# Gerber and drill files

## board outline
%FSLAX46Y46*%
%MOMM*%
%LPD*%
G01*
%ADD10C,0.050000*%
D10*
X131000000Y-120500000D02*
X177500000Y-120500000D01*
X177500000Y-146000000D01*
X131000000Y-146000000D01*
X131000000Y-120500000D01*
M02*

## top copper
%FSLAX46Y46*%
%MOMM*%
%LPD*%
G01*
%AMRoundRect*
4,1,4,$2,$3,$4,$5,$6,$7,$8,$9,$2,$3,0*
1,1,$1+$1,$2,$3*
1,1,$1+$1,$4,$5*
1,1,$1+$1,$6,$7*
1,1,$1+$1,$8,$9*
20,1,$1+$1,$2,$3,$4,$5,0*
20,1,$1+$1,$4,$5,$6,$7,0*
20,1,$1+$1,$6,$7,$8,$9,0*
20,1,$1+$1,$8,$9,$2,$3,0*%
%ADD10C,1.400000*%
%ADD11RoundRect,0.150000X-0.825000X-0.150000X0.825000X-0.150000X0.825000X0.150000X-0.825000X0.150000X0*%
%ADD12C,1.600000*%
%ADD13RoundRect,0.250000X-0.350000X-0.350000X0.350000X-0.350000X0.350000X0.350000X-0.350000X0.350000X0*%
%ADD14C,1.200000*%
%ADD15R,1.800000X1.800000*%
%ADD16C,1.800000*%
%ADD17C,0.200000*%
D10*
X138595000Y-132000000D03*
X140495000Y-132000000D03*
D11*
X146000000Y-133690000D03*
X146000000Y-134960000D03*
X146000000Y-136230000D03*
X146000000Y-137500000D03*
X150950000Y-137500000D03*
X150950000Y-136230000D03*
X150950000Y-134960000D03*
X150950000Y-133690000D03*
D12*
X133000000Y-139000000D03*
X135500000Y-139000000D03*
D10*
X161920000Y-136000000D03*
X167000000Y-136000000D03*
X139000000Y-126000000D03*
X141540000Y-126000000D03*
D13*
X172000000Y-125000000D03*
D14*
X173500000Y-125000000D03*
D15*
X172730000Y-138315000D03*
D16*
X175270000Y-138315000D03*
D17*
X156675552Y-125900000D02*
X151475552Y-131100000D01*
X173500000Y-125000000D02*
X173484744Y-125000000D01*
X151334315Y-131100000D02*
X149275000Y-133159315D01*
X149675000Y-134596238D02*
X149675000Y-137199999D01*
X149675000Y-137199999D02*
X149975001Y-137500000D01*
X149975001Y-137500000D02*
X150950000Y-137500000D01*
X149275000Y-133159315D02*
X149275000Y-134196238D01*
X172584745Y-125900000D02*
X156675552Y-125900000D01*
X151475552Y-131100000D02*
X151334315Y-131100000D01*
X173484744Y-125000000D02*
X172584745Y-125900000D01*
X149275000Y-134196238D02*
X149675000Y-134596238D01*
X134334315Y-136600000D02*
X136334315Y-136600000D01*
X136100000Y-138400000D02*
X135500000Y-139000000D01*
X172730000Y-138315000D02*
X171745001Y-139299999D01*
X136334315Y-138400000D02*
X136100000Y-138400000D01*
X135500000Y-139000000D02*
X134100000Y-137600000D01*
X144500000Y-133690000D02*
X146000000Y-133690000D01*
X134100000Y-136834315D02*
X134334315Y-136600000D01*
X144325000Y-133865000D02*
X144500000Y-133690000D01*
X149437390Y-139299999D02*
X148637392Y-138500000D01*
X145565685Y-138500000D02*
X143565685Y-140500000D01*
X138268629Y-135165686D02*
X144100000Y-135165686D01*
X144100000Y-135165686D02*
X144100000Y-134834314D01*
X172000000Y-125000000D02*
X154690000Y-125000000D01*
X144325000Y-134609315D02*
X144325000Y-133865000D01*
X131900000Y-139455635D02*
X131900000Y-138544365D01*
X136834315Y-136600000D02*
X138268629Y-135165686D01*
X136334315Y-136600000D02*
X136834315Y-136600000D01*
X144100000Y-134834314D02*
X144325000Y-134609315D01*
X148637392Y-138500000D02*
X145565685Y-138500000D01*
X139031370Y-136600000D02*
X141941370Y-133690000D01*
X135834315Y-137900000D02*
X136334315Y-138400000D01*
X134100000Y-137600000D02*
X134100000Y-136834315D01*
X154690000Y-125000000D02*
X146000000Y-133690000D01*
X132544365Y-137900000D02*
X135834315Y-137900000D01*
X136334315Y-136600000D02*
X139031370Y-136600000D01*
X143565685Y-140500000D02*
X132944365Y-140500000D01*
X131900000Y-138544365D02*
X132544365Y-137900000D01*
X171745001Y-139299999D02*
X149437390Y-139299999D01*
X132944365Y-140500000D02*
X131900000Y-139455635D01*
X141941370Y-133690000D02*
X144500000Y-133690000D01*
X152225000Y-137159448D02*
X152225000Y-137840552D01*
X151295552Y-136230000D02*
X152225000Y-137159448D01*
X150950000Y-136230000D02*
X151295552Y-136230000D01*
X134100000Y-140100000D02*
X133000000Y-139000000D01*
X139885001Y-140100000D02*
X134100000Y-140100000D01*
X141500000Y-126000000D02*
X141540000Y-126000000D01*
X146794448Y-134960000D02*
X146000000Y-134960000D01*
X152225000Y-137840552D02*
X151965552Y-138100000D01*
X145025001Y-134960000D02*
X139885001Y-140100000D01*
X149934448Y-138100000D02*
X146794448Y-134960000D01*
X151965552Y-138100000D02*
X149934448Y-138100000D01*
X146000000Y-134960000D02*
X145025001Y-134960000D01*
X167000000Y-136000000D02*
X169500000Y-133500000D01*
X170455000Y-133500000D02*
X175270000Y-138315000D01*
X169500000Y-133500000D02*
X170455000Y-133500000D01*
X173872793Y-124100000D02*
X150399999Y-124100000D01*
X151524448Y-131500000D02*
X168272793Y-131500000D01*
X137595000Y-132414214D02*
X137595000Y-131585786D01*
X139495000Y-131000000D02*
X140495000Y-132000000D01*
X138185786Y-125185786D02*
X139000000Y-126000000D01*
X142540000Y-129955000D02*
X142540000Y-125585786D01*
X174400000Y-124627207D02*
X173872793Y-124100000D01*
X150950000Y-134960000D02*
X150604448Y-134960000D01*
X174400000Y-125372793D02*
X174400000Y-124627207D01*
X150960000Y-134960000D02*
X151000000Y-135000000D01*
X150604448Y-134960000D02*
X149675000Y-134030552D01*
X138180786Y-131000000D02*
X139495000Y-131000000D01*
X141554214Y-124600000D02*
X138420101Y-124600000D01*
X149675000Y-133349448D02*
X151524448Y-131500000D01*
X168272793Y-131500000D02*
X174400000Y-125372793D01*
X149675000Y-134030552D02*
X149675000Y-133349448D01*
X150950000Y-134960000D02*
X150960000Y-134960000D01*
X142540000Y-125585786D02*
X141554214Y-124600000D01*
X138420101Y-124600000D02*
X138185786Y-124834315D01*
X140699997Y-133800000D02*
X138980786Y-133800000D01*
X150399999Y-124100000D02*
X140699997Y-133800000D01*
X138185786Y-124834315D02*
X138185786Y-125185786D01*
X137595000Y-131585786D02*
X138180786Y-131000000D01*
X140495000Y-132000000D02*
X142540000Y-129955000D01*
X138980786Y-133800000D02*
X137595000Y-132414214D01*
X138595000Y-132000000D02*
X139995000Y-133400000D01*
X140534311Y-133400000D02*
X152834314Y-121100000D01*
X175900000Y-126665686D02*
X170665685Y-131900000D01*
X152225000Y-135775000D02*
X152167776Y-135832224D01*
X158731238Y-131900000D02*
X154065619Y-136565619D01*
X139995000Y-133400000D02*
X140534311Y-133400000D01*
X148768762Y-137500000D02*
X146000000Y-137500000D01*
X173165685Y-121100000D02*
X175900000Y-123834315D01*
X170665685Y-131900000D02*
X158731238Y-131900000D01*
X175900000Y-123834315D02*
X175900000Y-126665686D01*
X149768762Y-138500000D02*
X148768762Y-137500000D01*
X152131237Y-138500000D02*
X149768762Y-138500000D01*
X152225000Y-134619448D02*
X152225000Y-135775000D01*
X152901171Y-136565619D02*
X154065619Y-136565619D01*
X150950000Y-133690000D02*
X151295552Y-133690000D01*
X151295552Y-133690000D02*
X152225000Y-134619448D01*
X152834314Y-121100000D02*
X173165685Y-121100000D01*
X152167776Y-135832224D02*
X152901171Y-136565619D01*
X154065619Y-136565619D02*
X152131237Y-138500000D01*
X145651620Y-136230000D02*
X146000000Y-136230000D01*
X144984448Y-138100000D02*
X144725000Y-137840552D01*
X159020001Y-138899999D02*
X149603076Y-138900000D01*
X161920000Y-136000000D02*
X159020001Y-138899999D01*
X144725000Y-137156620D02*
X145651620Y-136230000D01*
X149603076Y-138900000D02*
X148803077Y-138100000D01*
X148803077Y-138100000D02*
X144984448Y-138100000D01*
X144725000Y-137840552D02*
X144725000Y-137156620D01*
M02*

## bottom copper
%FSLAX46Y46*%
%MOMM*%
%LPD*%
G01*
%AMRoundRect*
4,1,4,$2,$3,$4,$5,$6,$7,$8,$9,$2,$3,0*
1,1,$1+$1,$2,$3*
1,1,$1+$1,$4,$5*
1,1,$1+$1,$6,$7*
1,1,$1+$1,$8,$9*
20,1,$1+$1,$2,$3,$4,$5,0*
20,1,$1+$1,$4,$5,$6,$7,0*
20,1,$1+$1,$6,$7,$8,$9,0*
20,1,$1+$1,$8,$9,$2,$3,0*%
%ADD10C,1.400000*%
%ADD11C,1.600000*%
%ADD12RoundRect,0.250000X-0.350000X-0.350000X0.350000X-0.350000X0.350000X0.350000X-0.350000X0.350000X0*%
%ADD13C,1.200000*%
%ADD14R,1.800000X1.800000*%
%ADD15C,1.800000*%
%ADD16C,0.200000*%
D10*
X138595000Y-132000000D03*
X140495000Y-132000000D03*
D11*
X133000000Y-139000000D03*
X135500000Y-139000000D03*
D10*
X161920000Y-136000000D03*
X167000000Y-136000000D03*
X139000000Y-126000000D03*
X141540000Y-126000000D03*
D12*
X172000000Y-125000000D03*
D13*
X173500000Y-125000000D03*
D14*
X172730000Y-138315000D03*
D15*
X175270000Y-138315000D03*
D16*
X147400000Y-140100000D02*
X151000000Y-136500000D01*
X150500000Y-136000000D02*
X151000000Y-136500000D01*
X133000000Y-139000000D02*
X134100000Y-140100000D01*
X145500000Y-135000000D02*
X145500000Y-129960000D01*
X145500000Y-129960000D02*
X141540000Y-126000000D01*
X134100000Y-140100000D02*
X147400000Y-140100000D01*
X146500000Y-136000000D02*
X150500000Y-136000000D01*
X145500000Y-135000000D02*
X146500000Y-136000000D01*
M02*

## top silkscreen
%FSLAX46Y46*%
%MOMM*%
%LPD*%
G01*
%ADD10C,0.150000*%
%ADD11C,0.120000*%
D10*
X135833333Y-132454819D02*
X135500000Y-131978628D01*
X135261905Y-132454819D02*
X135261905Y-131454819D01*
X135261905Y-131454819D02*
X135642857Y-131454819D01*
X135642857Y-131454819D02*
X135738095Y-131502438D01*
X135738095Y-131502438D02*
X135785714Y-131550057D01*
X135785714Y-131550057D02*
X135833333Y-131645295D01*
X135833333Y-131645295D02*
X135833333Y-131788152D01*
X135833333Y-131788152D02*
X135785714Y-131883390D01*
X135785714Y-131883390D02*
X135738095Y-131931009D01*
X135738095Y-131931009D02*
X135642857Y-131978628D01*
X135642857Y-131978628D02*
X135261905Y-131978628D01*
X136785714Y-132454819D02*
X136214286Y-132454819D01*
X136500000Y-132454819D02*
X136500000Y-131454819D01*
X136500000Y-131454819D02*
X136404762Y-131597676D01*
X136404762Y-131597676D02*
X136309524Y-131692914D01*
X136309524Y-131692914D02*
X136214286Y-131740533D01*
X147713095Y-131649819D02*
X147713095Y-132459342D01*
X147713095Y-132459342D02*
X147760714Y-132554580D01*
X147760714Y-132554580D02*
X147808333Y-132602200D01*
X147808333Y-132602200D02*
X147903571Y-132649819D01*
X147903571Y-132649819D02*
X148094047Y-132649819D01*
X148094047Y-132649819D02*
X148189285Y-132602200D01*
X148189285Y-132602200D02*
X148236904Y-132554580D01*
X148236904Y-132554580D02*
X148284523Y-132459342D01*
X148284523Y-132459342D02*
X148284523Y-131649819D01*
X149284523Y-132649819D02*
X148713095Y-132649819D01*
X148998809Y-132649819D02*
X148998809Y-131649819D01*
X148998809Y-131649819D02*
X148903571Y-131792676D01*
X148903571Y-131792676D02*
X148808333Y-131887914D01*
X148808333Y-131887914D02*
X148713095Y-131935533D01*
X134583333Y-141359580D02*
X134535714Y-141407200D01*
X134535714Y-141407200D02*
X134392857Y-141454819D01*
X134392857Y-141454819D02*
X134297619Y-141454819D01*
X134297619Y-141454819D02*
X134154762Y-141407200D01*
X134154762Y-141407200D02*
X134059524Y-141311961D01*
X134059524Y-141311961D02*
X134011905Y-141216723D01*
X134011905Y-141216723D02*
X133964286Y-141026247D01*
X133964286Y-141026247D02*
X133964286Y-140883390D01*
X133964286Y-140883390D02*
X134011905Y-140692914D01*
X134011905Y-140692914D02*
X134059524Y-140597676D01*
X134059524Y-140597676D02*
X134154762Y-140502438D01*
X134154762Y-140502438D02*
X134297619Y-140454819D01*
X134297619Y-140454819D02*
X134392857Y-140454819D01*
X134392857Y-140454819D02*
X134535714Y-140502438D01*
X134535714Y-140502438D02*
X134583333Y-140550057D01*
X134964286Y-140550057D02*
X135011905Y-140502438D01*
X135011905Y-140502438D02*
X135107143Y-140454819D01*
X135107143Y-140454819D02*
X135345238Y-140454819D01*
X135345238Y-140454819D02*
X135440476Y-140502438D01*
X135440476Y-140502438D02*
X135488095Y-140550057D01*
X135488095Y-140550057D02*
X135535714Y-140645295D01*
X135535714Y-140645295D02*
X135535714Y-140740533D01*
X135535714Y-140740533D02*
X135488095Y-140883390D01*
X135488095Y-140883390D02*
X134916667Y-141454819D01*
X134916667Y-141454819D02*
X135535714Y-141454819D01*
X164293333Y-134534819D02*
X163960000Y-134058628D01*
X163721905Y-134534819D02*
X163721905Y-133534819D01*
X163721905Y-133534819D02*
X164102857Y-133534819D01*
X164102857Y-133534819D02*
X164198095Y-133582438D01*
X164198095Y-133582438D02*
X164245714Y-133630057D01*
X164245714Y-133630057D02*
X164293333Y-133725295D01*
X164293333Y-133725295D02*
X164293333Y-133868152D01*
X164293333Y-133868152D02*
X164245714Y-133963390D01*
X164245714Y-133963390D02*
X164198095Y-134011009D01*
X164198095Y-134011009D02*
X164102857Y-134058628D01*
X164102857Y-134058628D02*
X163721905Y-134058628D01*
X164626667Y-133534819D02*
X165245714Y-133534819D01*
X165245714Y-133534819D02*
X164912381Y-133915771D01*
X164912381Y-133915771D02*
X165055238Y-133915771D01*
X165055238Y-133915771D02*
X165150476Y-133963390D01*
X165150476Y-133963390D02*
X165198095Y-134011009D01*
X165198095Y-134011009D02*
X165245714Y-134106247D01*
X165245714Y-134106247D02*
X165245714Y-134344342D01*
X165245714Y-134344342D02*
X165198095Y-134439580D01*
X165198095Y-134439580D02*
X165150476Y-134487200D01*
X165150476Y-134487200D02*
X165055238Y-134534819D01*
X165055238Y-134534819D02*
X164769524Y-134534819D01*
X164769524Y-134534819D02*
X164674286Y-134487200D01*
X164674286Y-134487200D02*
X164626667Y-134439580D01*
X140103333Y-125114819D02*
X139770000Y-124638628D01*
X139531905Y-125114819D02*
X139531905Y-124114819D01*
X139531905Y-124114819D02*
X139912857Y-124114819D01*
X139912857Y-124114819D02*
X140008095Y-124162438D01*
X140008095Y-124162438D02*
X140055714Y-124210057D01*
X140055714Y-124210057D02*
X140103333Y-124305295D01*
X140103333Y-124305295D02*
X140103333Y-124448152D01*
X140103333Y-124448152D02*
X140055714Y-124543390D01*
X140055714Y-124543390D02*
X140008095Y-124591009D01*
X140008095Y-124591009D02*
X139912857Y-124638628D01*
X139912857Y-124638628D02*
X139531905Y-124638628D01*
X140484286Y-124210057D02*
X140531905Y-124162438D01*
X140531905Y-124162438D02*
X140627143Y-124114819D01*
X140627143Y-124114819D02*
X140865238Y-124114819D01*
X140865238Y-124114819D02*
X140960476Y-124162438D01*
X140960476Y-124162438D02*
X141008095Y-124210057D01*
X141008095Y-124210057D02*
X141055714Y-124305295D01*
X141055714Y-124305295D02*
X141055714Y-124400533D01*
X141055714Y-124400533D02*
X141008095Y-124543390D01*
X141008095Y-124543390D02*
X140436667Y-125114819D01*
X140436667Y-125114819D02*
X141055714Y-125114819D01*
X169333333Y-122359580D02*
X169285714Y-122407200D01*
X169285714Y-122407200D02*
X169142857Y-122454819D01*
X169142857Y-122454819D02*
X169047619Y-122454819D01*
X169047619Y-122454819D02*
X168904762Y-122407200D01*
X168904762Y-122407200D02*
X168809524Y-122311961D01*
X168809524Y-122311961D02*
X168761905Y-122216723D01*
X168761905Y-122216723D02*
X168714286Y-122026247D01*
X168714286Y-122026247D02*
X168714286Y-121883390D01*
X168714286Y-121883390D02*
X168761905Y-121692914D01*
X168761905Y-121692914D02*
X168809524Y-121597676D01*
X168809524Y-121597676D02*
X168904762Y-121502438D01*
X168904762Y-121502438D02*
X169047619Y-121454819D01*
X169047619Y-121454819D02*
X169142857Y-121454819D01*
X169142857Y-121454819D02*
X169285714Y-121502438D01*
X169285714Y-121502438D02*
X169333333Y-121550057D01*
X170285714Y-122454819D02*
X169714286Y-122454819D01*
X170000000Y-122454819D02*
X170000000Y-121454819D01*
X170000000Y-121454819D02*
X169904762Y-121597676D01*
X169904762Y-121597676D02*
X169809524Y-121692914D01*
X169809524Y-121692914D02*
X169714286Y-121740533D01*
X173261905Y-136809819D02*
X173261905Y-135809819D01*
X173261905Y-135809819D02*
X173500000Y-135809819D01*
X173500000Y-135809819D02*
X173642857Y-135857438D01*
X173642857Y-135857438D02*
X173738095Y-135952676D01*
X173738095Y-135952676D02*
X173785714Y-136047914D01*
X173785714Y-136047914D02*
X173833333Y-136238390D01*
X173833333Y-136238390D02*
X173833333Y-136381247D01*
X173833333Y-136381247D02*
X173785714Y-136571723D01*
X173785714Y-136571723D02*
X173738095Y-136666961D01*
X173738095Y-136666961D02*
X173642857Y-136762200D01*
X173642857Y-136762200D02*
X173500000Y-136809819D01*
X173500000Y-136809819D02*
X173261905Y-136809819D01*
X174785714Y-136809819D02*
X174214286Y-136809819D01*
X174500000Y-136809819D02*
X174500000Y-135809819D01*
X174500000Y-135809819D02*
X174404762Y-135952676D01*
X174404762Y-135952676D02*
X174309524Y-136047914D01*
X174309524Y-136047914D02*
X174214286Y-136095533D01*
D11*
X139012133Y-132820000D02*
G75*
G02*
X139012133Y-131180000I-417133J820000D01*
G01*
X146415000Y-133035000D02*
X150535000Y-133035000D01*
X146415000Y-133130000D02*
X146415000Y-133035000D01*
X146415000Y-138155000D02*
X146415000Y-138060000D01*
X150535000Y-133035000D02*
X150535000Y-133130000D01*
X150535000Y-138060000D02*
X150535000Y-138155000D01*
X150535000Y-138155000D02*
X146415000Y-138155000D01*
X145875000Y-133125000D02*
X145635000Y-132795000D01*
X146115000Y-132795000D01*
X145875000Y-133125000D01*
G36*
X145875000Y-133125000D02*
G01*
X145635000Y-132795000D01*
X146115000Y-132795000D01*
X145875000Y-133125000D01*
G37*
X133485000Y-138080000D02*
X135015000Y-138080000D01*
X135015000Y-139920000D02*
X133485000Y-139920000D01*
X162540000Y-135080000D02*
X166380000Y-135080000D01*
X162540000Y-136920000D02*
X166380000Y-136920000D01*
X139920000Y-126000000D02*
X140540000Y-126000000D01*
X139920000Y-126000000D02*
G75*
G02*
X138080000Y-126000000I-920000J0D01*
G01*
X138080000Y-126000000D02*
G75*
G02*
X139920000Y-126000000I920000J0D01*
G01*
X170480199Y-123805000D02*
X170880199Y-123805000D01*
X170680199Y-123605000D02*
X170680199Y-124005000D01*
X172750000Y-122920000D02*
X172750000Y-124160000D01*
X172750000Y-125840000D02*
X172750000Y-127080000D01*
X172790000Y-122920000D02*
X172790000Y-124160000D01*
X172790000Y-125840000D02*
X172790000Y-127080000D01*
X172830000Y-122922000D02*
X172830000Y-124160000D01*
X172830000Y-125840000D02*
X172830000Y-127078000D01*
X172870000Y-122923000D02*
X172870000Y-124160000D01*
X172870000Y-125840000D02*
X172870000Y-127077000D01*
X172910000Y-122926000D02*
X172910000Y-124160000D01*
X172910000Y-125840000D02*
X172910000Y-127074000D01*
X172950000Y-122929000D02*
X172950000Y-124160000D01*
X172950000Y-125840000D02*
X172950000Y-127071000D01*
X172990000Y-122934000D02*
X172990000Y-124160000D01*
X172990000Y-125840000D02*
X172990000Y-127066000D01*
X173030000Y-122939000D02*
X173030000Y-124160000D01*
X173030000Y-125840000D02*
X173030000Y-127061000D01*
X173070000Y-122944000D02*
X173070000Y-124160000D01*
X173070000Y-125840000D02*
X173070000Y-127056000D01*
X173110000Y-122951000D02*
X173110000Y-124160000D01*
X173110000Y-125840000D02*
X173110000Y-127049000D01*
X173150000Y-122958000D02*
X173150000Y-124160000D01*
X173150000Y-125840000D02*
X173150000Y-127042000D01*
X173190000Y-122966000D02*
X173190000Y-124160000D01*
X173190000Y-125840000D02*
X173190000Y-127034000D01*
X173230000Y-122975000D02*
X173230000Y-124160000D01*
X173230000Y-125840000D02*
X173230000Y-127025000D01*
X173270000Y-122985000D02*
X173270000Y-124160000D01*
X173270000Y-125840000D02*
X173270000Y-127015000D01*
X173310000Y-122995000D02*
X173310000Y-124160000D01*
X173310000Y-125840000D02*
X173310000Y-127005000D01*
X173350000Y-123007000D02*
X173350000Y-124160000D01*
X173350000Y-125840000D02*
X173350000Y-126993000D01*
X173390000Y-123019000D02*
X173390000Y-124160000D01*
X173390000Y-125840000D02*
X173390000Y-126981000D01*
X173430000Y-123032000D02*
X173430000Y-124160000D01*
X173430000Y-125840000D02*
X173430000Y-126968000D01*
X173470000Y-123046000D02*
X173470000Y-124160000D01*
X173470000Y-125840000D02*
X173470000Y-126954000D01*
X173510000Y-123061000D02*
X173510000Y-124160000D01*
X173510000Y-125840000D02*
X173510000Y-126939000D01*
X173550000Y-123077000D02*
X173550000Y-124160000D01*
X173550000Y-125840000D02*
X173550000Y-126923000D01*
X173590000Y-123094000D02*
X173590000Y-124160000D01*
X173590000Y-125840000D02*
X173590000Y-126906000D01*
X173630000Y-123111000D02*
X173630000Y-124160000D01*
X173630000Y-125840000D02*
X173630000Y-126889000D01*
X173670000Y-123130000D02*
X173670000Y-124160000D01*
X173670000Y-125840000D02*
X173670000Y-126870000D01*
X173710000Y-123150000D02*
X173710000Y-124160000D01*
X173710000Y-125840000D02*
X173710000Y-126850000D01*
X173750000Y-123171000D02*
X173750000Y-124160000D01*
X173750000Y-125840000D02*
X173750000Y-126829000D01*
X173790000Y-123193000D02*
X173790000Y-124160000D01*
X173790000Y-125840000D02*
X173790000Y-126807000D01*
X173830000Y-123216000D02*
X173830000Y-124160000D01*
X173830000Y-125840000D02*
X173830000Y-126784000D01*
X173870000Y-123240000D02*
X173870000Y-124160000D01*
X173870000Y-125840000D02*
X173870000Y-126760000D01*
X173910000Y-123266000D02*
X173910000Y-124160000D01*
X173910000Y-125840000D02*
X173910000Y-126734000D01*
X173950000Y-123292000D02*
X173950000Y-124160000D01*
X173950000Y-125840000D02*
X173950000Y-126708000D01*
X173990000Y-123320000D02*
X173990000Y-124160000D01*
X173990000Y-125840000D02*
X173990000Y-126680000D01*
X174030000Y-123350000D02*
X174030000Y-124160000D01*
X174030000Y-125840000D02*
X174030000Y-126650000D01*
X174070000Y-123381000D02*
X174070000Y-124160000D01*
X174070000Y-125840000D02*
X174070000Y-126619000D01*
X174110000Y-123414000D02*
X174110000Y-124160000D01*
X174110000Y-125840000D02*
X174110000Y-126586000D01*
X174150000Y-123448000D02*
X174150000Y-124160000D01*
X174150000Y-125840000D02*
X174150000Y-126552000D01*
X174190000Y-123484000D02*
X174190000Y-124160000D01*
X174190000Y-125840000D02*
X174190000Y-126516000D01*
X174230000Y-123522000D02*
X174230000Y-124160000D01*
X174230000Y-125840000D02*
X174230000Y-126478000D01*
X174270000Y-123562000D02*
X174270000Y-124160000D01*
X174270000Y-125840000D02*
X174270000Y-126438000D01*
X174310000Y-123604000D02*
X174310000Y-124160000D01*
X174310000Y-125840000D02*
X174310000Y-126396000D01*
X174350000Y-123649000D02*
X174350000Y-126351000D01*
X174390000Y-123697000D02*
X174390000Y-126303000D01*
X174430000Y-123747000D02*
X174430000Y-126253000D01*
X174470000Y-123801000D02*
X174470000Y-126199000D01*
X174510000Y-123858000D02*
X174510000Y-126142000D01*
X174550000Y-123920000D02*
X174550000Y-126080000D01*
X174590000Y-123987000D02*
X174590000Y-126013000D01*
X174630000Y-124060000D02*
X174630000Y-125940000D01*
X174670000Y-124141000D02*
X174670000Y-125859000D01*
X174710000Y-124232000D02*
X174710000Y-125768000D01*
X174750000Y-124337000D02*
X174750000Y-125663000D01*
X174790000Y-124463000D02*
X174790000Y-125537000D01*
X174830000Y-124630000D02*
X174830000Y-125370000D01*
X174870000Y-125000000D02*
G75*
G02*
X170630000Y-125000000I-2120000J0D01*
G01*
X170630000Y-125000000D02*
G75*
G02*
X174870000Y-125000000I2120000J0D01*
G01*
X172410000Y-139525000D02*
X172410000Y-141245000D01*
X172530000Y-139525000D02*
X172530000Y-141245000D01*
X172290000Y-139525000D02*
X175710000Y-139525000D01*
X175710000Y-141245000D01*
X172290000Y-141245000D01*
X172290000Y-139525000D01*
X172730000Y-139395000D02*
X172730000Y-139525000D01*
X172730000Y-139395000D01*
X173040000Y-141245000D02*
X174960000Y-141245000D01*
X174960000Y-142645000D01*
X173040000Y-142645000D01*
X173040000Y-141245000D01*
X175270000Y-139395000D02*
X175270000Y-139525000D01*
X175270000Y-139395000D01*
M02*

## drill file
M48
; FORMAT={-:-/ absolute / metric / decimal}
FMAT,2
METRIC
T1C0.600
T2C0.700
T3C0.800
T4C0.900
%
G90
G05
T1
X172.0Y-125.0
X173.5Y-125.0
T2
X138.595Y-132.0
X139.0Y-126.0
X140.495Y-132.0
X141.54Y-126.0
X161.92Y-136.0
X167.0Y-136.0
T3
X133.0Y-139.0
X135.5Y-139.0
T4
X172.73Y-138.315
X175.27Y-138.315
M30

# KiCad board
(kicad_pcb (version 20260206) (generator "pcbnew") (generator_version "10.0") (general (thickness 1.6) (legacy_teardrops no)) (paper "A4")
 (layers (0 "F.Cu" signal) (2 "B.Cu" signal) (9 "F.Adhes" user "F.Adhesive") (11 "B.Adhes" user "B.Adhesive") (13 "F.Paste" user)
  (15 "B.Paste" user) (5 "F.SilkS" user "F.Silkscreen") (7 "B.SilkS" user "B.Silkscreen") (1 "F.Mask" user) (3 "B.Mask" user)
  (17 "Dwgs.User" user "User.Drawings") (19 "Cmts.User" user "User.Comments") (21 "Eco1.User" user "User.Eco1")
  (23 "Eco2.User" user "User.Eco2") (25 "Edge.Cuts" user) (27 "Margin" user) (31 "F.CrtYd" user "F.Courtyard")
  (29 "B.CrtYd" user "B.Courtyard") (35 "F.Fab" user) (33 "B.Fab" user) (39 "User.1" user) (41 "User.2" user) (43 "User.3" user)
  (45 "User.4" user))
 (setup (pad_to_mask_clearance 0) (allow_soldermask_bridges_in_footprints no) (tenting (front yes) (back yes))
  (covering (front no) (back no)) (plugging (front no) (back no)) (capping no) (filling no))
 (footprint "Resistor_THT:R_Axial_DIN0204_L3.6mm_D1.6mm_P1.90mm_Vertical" (layer "F.Cu") (at 138.595 132)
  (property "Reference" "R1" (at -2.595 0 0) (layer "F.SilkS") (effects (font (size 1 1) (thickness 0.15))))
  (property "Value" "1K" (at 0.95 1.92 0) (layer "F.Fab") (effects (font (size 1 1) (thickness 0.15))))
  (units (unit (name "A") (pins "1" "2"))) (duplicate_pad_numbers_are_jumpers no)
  (fp_arc (start 0.417133 0.82) (mid -0.92 0) (end 0.417133 -0.82) (stroke (width 0.12) (type solid)) (layer "F.SilkS"))
  (pad "1" thru_hole circle (at 0 0) (size 1.4 1.4) (drill 0.7) (layers "*.Cu" "*.Mask") (remove_unused_layers no) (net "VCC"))
  (pad "2" thru_hole circle (at 1.9 0) (size 1.4 1.4) (drill 0.7) (layers "*.Cu" "*.Mask") (remove_unused_layers no) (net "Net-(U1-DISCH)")))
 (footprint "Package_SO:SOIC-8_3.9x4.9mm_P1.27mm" (layer "F.Cu") (at 148.475 135.595)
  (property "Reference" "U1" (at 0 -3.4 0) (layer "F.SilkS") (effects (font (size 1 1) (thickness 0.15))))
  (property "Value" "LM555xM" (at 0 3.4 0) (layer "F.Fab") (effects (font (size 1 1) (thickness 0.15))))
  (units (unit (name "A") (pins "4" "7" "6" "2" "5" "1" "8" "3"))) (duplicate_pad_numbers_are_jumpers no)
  (fp_line (start -2.06 -2.56) (end 2.06 -2.56) (stroke (width 0.12) (type solid)) (layer "F.SilkS"))
  (fp_line (start -2.06 -2.465) (end -2.06 -2.56) (stroke (width 0.12) (type solid)) (layer "F.SilkS"))
  (fp_line (start -2.06 2.56) (end -2.06 2.465) (stroke (width 0.12) (type solid)) (layer "F.SilkS"))
  (fp_line (start 2.06 -2.56) (end 2.06 -2.465) (stroke (width 0.12) (type solid)) (layer "F.SilkS"))
  (fp_line (start 2.06 2.465) (end 2.06 2.56) (stroke (width 0.12) (type solid)) (layer "F.SilkS"))
  (fp_line (start 2.06 2.56) (end -2.06 2.56) (stroke (width 0.12) (type solid)) (layer "F.SilkS"))
  (fp_poly (pts (xy -2.6 -2.47) (xy -2.84 -2.8) (xy -2.36 -2.8)) (stroke (width 0.12) (type solid)) (fill yes) (layer "F.SilkS"))
  (pad "1" smd roundrect (at -2.475 -1.905) (size 1.95 0.6) (layers "F.Cu" "F.Mask" "F.Paste") (roundrect_rratio 0.25) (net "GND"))
  (pad "2" smd roundrect (at -2.475 -0.635) (size 1.95 0.6) (layers "F.Cu" "F.Mask" "F.Paste") (roundrect_rratio 0.25)
   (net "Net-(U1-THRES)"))
  (pad "3" smd roundrect (at -2.475 0.635) (size 1.95 0.6) (layers "F.Cu" "F.Mask" "F.Paste") (roundrect_rratio 0.25) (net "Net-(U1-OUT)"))
  (pad "4" smd roundrect (at -2.475 1.905) (size 1.95 0.6) (layers "F.Cu" "F.Mask" "F.Paste") (roundrect_rratio 0.25) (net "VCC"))
  (pad "5" smd roundrect (at 2.475 1.905) (size 1.95 0.6) (layers "F.Cu" "F.Mask" "F.Paste") (roundrect_rratio 0.25) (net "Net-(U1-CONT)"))
  (pad "6" smd roundrect (at 2.475 0.635) (size 1.95 0.6) (layers "F.Cu" "F.Mask" "F.Paste") (roundrect_rratio 0.25) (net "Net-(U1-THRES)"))
  (pad "7" smd roundrect (at 2.475 -0.635) (size 1.95 0.6) (layers "F.Cu" "F.Mask" "F.Paste") (roundrect_rratio 0.25) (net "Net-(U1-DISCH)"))
  (pad "8" smd roundrect (at 2.475 -1.905) (size 1.95 0.6) (layers "F.Cu" "F.Mask" "F.Paste") (roundrect_rratio 0.25) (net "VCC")))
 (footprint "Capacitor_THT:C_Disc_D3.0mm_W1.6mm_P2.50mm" (layer "F.Cu") (at 133 139)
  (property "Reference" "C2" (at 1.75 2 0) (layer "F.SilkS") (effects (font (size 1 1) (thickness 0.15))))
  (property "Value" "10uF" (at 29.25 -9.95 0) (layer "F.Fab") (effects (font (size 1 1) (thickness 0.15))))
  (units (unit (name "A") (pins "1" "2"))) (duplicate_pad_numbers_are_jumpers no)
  (fp_line (start 0.485 -0.92) (end 2.015 -0.92) (stroke (width 0.12) (type solid)) (layer "F.SilkS"))
  (fp_line (start 2.015 0.92) (end 0.485 0.92) (stroke (width 0.12) (type solid)) (layer "F.SilkS"))
  (pad "1" thru_hole circle (at 0 0) (size 1.6 1.6) (drill 0.8) (layers "*.Cu" "*.Mask") (remove_unused_layers no) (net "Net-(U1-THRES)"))
  (pad "2" thru_hole circle (at 2.5 0) (size 1.6 1.6) (drill 0.8) (layers "*.Cu" "*.Mask") (remove_unused_layers no) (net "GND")))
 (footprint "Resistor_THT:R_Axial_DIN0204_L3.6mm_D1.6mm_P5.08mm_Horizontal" (layer "F.Cu") (at 161.92 136)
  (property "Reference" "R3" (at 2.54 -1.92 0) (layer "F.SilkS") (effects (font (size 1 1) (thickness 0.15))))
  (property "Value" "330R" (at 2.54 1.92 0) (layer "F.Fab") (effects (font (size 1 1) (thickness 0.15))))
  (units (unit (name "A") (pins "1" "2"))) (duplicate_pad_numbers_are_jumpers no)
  (fp_line (start 0.62 -0.92) (end 4.46 -0.92) (stroke (width 0.12) (type solid)) (layer "F.SilkS"))
  (fp_line (start 0.62 0.92) (end 4.46 0.92) (stroke (width 0.12) (type solid)) (layer "F.SilkS"))
  (pad "1" thru_hole circle (at 0 0) (size 1.4 1.4) (drill 0.7) (layers "*.Cu" "*.Mask") (remove_unused_layers no) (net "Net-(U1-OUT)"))
  (pad "2" thru_hole circle (at 5.08 0) (size 1.4 1.4) (drill 0.7) (layers "*.Cu" "*.Mask") (remove_unused_layers no) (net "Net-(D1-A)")))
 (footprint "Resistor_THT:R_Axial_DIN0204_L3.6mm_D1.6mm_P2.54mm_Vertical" (layer "F.Cu") (at 139 126)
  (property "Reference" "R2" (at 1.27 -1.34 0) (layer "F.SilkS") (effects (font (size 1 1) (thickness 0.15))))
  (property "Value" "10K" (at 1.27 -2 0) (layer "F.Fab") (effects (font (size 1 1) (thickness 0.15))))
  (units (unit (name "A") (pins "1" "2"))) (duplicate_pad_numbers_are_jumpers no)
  (fp_line (start 0.92 0) (end 1.54 0) (stroke (width 0.12) (type solid)) (layer "F.SilkS"))
  (fp_circle (center 0 0) (end 0.92 0) (stroke (width 0.12) (type solid)) (fill no) (layer "F.SilkS"))
  (pad "1" thru_hole circle (at 0 0) (size 1.4 1.4) (drill 0.7) (layers "*.Cu" "*.Mask") (remove_unused_layers no) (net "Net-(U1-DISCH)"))
  (pad "2" thru_hole circle (at 2.54 0) (size 1.4 1.4) (drill 0.7) (layers "*.Cu" "*.Mask") (remove_unused_layers no) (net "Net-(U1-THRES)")))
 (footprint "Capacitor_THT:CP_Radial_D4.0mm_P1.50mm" (layer "F.Cu") (at 172 125)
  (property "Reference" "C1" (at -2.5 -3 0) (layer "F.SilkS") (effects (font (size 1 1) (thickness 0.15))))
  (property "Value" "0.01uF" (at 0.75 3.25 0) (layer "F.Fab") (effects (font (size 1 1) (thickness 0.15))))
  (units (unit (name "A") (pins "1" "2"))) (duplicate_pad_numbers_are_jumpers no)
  (fp_line (start -1.519801 -1.195) (end -1.119801 -1.195) (stroke (width 0.12) (type solid)) (layer "F.SilkS"))
  (fp_line (start -1.319801 -1.395) (end -1.319801 -0.995) (stroke (width 0.12) (type solid)) (layer "F.SilkS"))
  (fp_line (start 0.75 -2.08) (end 0.75 -0.84) (stroke (width 0.12) (type solid)) (layer "F.SilkS"))
  (fp_line (start 0.75 0.84) (end 0.75 2.08) (stroke (width 0.12) (type solid)) (layer "F.SilkS"))
  (fp_line (start 0.79 -2.08) (end 0.79 -0.84) (stroke (width 0.12) (type solid)) (layer "F.SilkS"))
  (fp_line (start 0.79 0.84) (end 0.79 2.08) (stroke (width 0.12) (type solid)) (layer "F.SilkS"))
  (fp_line (start 0.83 -2.078) (end 0.83 -0.84) (stroke (width 0.12) (type solid)) (layer "F.SilkS"))
  (fp_line (start 0.83 0.84) (end 0.83 2.078) (stroke (width 0.12) (type solid)) (layer "F.SilkS"))
  (fp_line (start 0.87 -2.077) (end 0.87 -0.84) (stroke (width 0.12) (type solid)) (layer "F.SilkS"))
  (fp_line (start 0.87 0.84) (end 0.87 2.077) (stroke (width 0.12) (type solid)) (layer "F.SilkS"))
  (fp_line (start 0.91 -2.074) (end 0.91 -0.84) (stroke (width 0.12) (type solid)) (layer "F.SilkS"))
  (fp_line (start 0.91 0.84) (end 0.91 2.074) (stroke (width 0.12) (type solid)) (layer "F.SilkS"))
  (fp_line (start 0.95 -2.071) (end 0.95 -0.84) (stroke (width 0.12) (type solid)) (layer "F.SilkS"))
  (fp_line (start 0.95 0.84) (end 0.95 2.071) (stroke (width 0.12) (type solid)) (layer "F.SilkS"))
  (fp_line (start 0.99 -2.066) (end 0.99 -0.84) (stroke (width 0.12) (type solid)) (layer "F.SilkS"))
  (fp_line (start 0.99 0.84) (end 0.99 2.066) (stroke (width 0.12) (type solid)) (layer "F.SilkS"))
  (fp_line (start 1.03 -2.061) (end 1.03 -0.84) (stroke (width 0.12) (type solid)) (layer "F.SilkS"))
  (fp_line (start 1.03 0.84) (end 1.03 2.061) (stroke (width 0.12) (type solid)) (layer "F.SilkS"))
  (fp_line (start 1.07 -2.056) (end 1.07 -0.84) (stroke (width 0.12) (type solid)) (layer "F.SilkS"))
  (fp_line (start 1.07 0.84) (end 1.07 2.056) (stroke (width 0.12) (type solid)) (layer "F.SilkS"))
  (fp_line (start 1.11 -2.049) (end 1.11 -0.84) (stroke (width 0.12) (type solid)) (layer "F.SilkS"))
  (fp_line (start 1.11 0.84) (end 1.11 2.049) (stroke (width 0.12) (type solid)) (layer "F.SilkS"))
  (fp_line (start 1.15 -2.042) (end 1.15 -0.84) (stroke (width 0.12) (type solid)) (layer "F.SilkS"))
  (fp_line (start 1.15 0.84) (end 1.15 2.042) (stroke (width 0.12) (type solid)) (layer "F.SilkS"))
  (fp_line (start 1.19 -2.034) (end 1.19 -0.84) (stroke (width 0.12) (type solid)) (layer "F.SilkS"))
  (fp_line (start 1.19 0.84) (end 1.19 2.034) (stroke (width 0.12) (type solid)) (layer "F.SilkS"))
  (fp_line (start 1.23 -2.025) (end 1.23 -0.84) (stroke (width 0.12) (type solid)) (layer "F.SilkS"))
  (fp_line (start 1.23 0.84) (end 1.23 2.025) (stroke (width 0.12) (type solid)) (layer "F.SilkS"))
  (fp_line (start 1.27 -2.015) (end 1.27 -0.84) (stroke (width 0.12) (type solid)) (layer "F.SilkS"))
  (fp_line (start 1.27 0.84) (end 1.27 2.015) (stroke (width 0.12) (type solid)) (layer "F.SilkS"))
  (fp_line (start 1.31 -2.005) (end 1.31 -0.84) (stroke (width 0.12) (type solid)) (layer "F.SilkS"))
  (fp_line (start 1.31 0.84) (end 1.31 2.005) (stroke (width 0.12) (type solid)) (layer "F.SilkS"))
  (fp_line (start 1.35 -1.993) (end 1.35 -0.84) (stroke (width 0.12) (type solid)) (layer "F.SilkS"))
  (fp_line (start 1.35 0.84) (end 1.35 1.993) (stroke (width 0.12) (type solid)) (layer "F.SilkS"))
  (fp_line (start 1.39 -1.981) (end 1.39 -0.84) (stroke (width 0.12) (type solid)) (layer "F.SilkS"))
  (fp_line (start 1.39 0.84) (end 1.39 1.981) (stroke (width 0.12) (type solid)) (layer "F.SilkS"))
  (fp_line (start 1.43 -1.968) (end 1.43 -0.84) (stroke (width 0.12) (type solid)) (layer "F.SilkS"))
  (fp_line (start 1.43 0.84) (end 1.43 1.968) (stroke (width 0.12) (type solid)) (layer "F.SilkS"))
  (fp_line (start 1.47 -1.954) (end 1.47 -0.84) (stroke (width 0.12) (type solid)) (layer "F.SilkS"))
  (fp_line (start 1.47 0.84) (end 1.47 1.954) (stroke (width 0.12) (type solid)) (layer "F.SilkS"))
  (fp_line (start 1.51 -1.939) (end 1.51 -0.84) (stroke (width 0.12) (type solid)) (layer "F.SilkS"))
  (fp_line (start 1.51 0.84) (end 1.51 1.939) (stroke (width 0.12) (type solid)) (layer "F.SilkS"))
  (fp_line (start 1.55 -1.923) (end 1.55 -0.84) (stroke (width 0.12) (type solid)) (layer "F.SilkS"))
  (fp_line (start 1.55 0.84) (end 1.55 1.923) (stroke (width 0.12) (type solid)) (layer "F.SilkS"))
  (fp_line (start 1.59 -1.906) (end 1.59 -0.84) (stroke (width 0.12) (type solid)) (layer "F.SilkS"))
  (fp_line (start 1.59 0.84) (end 1.59 1.906) (stroke (width 0.12) (type solid)) (layer "F.SilkS"))
  (fp_line (start 1.63 -1.889) (end 1.63 -0.84) (stroke (width 0.12) (type solid)) (layer "F.SilkS"))
  (fp_line (start 1.63 0.84) (end 1.63 1.889) (stroke (width 0.12) (type solid)) (layer "F.SilkS"))
  (fp_line (start 1.67 -1.87) (end 1.67 -0.84) (stroke (width 0.12) (type solid)) (layer "F.SilkS"))
  (fp_line (start 1.67 0.84) (end 1.67 1.87) (stroke (width 0.12) (type solid)) (layer "F.SilkS"))
  (fp_line (start 1.71 -1.85) (end 1.71 -0.84) (stroke (width 0.12) (type solid)) (layer "F.SilkS"))
  (fp_line (start 1.71 0.84) (end 1.71 1.85) (stroke (width 0.12) (type solid)) (layer "F.SilkS"))
  (fp_line (start 1.75 -1.829) (end 1.75 -0.84) (stroke (width 0.12) (type solid)) (layer "F.SilkS"))
  (fp_line (start 1.75 0.84) (end 1.75 1.829) (stroke (width 0.12) (type solid)) (layer "F.SilkS"))
  (fp_line (start 1.79 -1.807) (end 1.79 -0.84) (stroke (width 0.12) (type solid)) (layer "F.SilkS"))
  (fp_line (start 1.79 0.84) (end 1.79 1.807) (stroke (width 0.12) (type solid)) (layer "F.SilkS"))
  (fp_line (start 1.83 -1.784) (end 1.83 -0.84) (stroke (width 0.12) (type solid)) (layer "F.SilkS"))
  (fp_line (start 1.83 0.84) (end 1.83 1.784) (stroke (width 0.12) (type solid)) (layer "F.SilkS"))
  (fp_line (start 1.87 -1.76) (end 1.87 -0.84) (stroke (width 0.12) (type solid)) (layer "F.SilkS"))
  (fp_line (start 1.87 0.84) (end 1.87 1.76) (stroke (width 0.12) (type solid)) (layer "F.SilkS"))
  (fp_line (start 1.91 -1.734) (end 1.91 -0.84) (stroke (width 0.12) (type solid)) (layer "F.SilkS"))
  (fp_line (start 1.91 0.84) (end 1.91 1.734) (stroke (width 0.12) (type solid)) (layer "F.SilkS"))
  (fp_line (start 1.95 -1.708) (end 1.95 -0.84) (stroke (width 0.12) (type solid)) (layer "F.SilkS"))
  (fp_line (start 1.95 0.84) (end 1.95 1.708) (stroke (width 0.12) (type solid)) (layer "F.SilkS"))
  (fp_line (start 1.99 -1.68) (end 1.99 -0.84) (stroke (width 0.12) (type solid)) (layer "F.SilkS"))
  (fp_line (start 1.99 0.84) (end 1.99 1.68) (stroke (width 0.12) (type solid)) (layer "F.SilkS"))
  (fp_line (start 2.03 -1.65) (end 2.03 -0.84) (stroke (width 0.12) (type solid)) (layer "F.SilkS"))
  (fp_line (start 2.03 0.84) (end 2.03 1.65) (stroke (width 0.12) (type solid)) (layer "F.SilkS"))
  (fp_line (start 2.07 -1.619) (end 2.07 -0.84) (stroke (width 0.12) (type solid)) (layer "F.SilkS"))
  (fp_line (start 2.07 0.84) (end 2.07 1.619) (stroke (width 0.12) (type solid)) (layer "F.SilkS"))
  (fp_line (start 2.11 -1.586) (end 2.11 -0.84) (stroke (width 0.12) (type solid)) (layer "F.SilkS"))
  (fp_line (start 2.11 0.84) (end 2.11 1.586) (stroke (width 0.12) (type solid)) (layer "F.SilkS"))
  (fp_line (start 2.15 -1.552) (end 2.15 -0.84) (stroke (width 0.12) (type solid)) (layer "F.SilkS"))
  (fp_line (start 2.15 0.84) (end 2.15 1.552) (stroke (width 0.12) (type solid)) (layer "F.SilkS"))
  (fp_line (start 2.19 -1.516) (end 2.19 -0.84) (stroke (width 0.12) (type solid)) (layer "F.SilkS"))
  (fp_line (start 2.19 0.84) (end 2.19 1.516) (stroke (width 0.12) (type solid)) (layer "F.SilkS"))
  (fp_line (start 2.23 -1.478) (end 2.23 -0.84) (stroke (width 0.12) (type solid)) (layer "F.SilkS"))
  (fp_line (start 2.23 0.84) (end 2.23 1.478) (stroke (width 0.12) (type solid)) (layer "F.SilkS"))
  (fp_line (start 2.27 -1.438) (end 2.27 -0.84) (stroke (width 0.12) (type solid)) (layer "F.SilkS"))
  (fp_line (start 2.27 0.84) (end 2.27 1.438) (stroke (width 0.12) (type solid)) (layer "F.SilkS"))
  (fp_line (start 2.31 -1.396) (end 2.31 -0.84) (stroke (width 0.12) (type solid)) (layer "F.SilkS"))
  (fp_line (start 2.31 0.84) (end 2.31 1.396) (stroke (width 0.12) (type solid)) (layer "F.SilkS"))
  (fp_line (start 2.35 -1.351) (end 2.35 1.351) (stroke (width 0.12) (type solid)) (layer "F.SilkS"))
  (fp_line (start 2.39 -1.303) (end 2.39 1.303) (stroke (width 0.12) (type solid)) (layer "F.SilkS"))
  (fp_line (start 2.43 -1.253) (end 2.43 1.253) (stroke (width 0.12) (type solid)) (layer "F.SilkS"))
  (fp_line (start 2.47 -1.199) (end 2.47 1.199) (stroke (width 0.12) (type solid)) (layer "F.SilkS"))
  (fp_line (start 2.51 -1.142) (end 2.51 1.142) (stroke (width 0.12) (type solid)) (layer "F.SilkS"))
  (fp_line (start 2.55 -1.08) (end 2.55 1.08) (stroke (width 0.12) (type solid)) (layer "F.SilkS"))
  (fp_line (start 2.59 -1.013) (end 2.59 1.013) (stroke (width 0.12) (type solid)) (layer "F.SilkS"))
  (fp_line (start 2.63 -0.94) (end 2.63 0.94) (stroke (width 0.12) (type solid)) (layer "F.SilkS"))
  (fp_line (start 2.67 -0.859) (end 2.67 0.859) (stroke (width 0.12) (type solid)) (layer "F.SilkS"))
  (fp_line (start 2.71 -0.768) (end 2.71 0.768) (stroke (width 0.12) (type solid)) (layer "F.SilkS"))
  (fp_line (start 2.75 -0.663) (end 2.75 0.663) (stroke (width 0.12) (type solid)) (layer "F.SilkS"))
  (fp_line (start 2.79 -0.537) (end 2.79 0.537) (stroke (width 0.12) (type solid)) (layer "F.SilkS"))
  (fp_line (start 2.83 -0.37) (end 2.83 0.37) (stroke (width 0.12) (type solid)) (layer "F.SilkS"))
  (fp_circle (center 0.75 0) (end 2.87 0) (stroke (width 0.12) (type solid)) (fill no) (layer "F.SilkS"))
  (pad "1" thru_hole roundrect (at 0 0) (size 1.2 1.2) (drill 0.6) (layers "*.Cu" "*.Mask") (remove_unused_layers no)
   (roundrect_rratio 0.208333) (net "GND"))
  (pad "2" thru_hole circle (at 1.5 0) (size 1.2 1.2) (drill 0.6) (layers "*.Cu" "*.Mask") (remove_unused_layers no) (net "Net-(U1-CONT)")))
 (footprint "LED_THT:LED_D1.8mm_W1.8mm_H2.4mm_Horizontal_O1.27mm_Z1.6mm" (layer "F.Cu") (at 172.73 138.315)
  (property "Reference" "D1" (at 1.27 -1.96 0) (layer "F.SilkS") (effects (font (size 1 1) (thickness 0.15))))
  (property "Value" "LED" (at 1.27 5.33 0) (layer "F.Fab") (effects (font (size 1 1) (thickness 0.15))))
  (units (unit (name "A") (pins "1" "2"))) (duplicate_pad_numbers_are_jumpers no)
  (fp_line (start -0.32 1.21) (end -0.32 2.93) (stroke (width 0.12) (type solid)) (layer "F.SilkS"))
  (fp_line (start -0.2 1.21) (end -0.2 2.93) (stroke (width 0.12) (type solid)) (layer "F.SilkS"))
  (fp_rect (start -0.44 1.21) (end 2.98 2.93) (stroke (width 0.12) (type solid)) (fill no) (layer "F.SilkS"))
  (fp_rect (start 0 1.08) (end 0 1.21) (stroke (width 0.12) (type solid)) (fill no) (layer "F.SilkS"))
  (fp_rect (start 0.31 2.93) (end 2.23 4.33) (stroke (width 0.12) (type solid)) (fill no) (layer "F.SilkS"))
  (fp_rect (start 2.54 1.08) (end 2.54 1.21) (stroke (width 0.12) (type solid)) (fill no) (layer "F.SilkS"))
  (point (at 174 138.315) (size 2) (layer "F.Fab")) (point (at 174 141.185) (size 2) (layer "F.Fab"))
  (pad "1" thru_hole rect (at 0 0) (size 1.8 1.8) (drill 0.9) (layers "*.Cu" "*.Mask") (remove_unused_layers no) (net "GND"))
  (pad "2" thru_hole circle (at 2.54 0) (size 1.8 1.8) (drill 0.9) (layers "*.Cu" "*.Mask") (remove_unused_layers no) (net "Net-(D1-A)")))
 (gr_rect (start 131 120.5) (end 177.5 146) (stroke (width 0.05) (type default)) (fill no) (layer "Edge.Cuts"))
 (segment (start 156.675552 125.9) (end 151.475552 131.1) (width 0.2) (layer "F.Cu") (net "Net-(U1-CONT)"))
 (segment (start 173.5 125) (end 173.484744 125) (width 0.2) (layer "F.Cu") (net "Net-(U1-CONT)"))
 (segment (start 151.334315 131.1) (end 149.275 133.159315) (width 0.2) (layer "F.Cu") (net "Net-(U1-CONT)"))
 (segment (start 149.675 134.596238) (end 149.675 137.199999) (width 0.2) (layer "F.Cu") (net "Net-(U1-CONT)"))
 (segment (start 149.675 137.199999) (end 149.975001 137.5) (width 0.2) (layer "F.Cu") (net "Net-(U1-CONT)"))
 (segment (start 149.975001 137.5) (end 150.95 137.5) (width 0.2) (layer "F.Cu") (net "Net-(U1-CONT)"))
 (segment (start 149.275 133.159315) (end 149.275 134.196238) (width 0.2) (layer "F.Cu") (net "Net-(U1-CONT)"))
 (segment (start 172.584745 125.9) (end 156.675552 125.9) (width 0.2) (layer "F.Cu") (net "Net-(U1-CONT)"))
 (segment (start 151.475552 131.1) (end 151.334315 131.1) (width 0.2) (layer "F.Cu") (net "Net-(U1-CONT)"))
 (segment (start 173.484744 125) (end 172.584745 125.9) (width 0.2) (layer "F.Cu") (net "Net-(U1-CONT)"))
 (segment (start 149.275 134.196238) (end 149.675 134.596238) (width 0.2) (layer "F.Cu") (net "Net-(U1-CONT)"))
 (segment (start 134.334315 136.6) (end 136.334315 136.6) (width 0.2) (layer "F.Cu") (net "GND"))
 (segment (start 136.1 138.4) (end 135.5 139) (width 0.2) (layer "F.Cu") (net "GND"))
 (segment (start 172.73 138.315) (end 171.745001 139.299999) (width 0.2) (layer "F.Cu") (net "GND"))
 (segment (start 136.334315 138.4) (end 136.1 138.4) (width 0.2) (layer "F.Cu") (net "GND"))
 (segment (start 135.5 139) (end 134.1 137.6) (width 0.2) (layer "F.Cu") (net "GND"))
 (segment (start 144.5 133.69) (end 146 133.69) (width 0.2) (layer "F.Cu") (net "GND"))
 (segment (start 134.1 136.834315) (end 134.334315 136.6) (width 0.2) (layer "F.Cu") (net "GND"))
 (segment (start 144.325 133.865) (end 144.5 133.69) (width 0.2) (layer "F.Cu") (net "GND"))
 (segment (start 149.43739 139.299999) (end 148.637392 138.5) (width 0.2) (layer "F.Cu") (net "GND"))
 (segment (start 145.565685 138.5) (end 143.565685 140.5) (width 0.2) (layer "F.Cu") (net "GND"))
 (segment (start 138.268629 135.165686) (end 144.1 135.165686) (width 0.2) (layer "F.Cu") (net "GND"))
 (segment (start 144.1 135.165686) (end 144.1 134.834314) (width 0.2) (layer "F.Cu") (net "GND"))
 (segment (start 172 125) (end 154.69 125) (width 0.2) (layer "F.Cu") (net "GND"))
 (segment (start 144.325 134.609315) (end 144.325 133.865) (width 0.2) (layer "F.Cu") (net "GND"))
 (segment (start 131.9 139.455635) (end 131.9 138.544365) (width 0.2) (layer "F.Cu") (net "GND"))
 (segment (start 136.834315 136.6) (end 138.268629 135.165686) (width 0.2) (layer "F.Cu") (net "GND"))
 (segment (start 136.334315 136.6) (end 136.834315 136.6) (width 0.2) (layer "F.Cu") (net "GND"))
 (segment (start 144.1 134.834314) (end 144.325 134.609315) (width 0.2) (layer "F.Cu") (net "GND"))
 (segment (start 148.637392 138.5) (end 145.565685 138.5) (width 0.2) (layer "F.Cu") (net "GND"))
 (segment (start 139.03137 136.6) (end 141.94137 133.69) (width 0.2) (layer "F.Cu") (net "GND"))
 (segment (start 135.834315 137.9) (end 136.334315 138.4) (width 0.2) (layer "F.Cu") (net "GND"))
 (segment (start 134.1 137.6) (end 134.1 136.834315) (width 0.2) (layer "F.Cu") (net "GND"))
 (segment (start 154.69 125) (end 146 133.69) (width 0.2) (layer "F.Cu") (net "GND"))
 (segment (start 132.544365 137.9) (end 135.834315 137.9) (width 0.2) (layer "F.Cu") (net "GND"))
 (segment (start 136.334315 136.6) (end 139.03137 136.6) (width 0.2) (layer "F.Cu") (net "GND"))
 (segment (start 143.565685 140.5) (end 132.944365 140.5) (width 0.2) (layer "F.Cu") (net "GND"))
 (segment (start 131.9 138.544365) (end 132.544365 137.9) (width 0.2) (layer "F.Cu") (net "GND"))
 (segment (start 171.745001 139.299999) (end 149.43739 139.299999) (width 0.2) (layer "F.Cu") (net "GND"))
 (segment (start 132.944365 140.5) (end 131.9 139.455635) (width 0.2) (layer "F.Cu") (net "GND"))
 (segment (start 141.94137 133.69) (end 144.5 133.69) (width 0.2) (layer "F.Cu") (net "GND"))
 (segment (start 152.225 137.159448) (end 152.225 137.840552) (width 0.2) (layer "F.Cu") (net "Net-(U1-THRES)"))
 (segment (start 151.295552 136.23) (end 152.225 137.159448) (width 0.2) (layer "F.Cu") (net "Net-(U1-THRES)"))
 (segment (start 150.95 136.23) (end 151.295552 136.23) (width 0.2) (layer "F.Cu") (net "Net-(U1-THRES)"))
 (segment (start 134.1 140.1) (end 133 139) (width 0.2) (layer "F.Cu") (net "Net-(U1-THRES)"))
 (segment (start 139.885001 140.1) (end 134.1 140.1) (width 0.2) (layer "F.Cu") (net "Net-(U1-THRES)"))
 (segment (start 141.5 126) (end 141.54 126) (width 0.2) (layer "F.Cu") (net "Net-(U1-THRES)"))
 (segment (start 146.794448 134.96) (end 146 134.96) (width 0.2) (layer "F.Cu") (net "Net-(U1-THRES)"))
 (segment (start 152.225 137.840552) (end 151.965552 138.1) (width 0.2) (layer "F.Cu") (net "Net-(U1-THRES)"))
 (segment (start 145.025001 134.96) (end 139.885001 140.1) (width 0.2) (layer "F.Cu") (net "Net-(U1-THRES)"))
 (segment (start 149.934448 138.1) (end 146.794448 134.96) (width 0.2) (layer "F.Cu") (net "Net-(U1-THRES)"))
 (segment (start 151.965552 138.1) (end 149.934448 138.1) (width 0.2) (layer "F.Cu") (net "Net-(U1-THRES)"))
 (segment (start 146 134.96) (end 145.025001 134.96) (width 0.2) (layer "F.Cu") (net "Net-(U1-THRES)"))
 (segment (start 147.4 140.1) (end 151 136.5) (width 0.2) (layer "B.Cu") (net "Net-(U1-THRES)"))
 (segment (start 150.5 136) (end 151 136.5) (width 0.2) (layer "B.Cu") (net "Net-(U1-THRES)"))
 (segment (start 133 139) (end 134.1 140.1) (width 0.2) (layer "B.Cu") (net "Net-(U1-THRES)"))
 (segment (start 145.5 135) (end 145.5 129.96) (width 0.2) (layer "B.Cu") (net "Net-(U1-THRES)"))
 (segment (start 145.5 129.96) (end 141.54 126) (width 0.2) (layer "B.Cu") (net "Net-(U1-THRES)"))
 (segment (start 134.1 140.1) (end 147.4 140.1) (width 0.2) (layer "B.Cu") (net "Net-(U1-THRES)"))
 (segment (start 146.5 136) (end 150.5 136) (width 0.2) (layer "B.Cu") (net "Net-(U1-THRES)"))
 (segment (start 145.5 135) (end 146.5 136) (width 0.2) (layer "B.Cu") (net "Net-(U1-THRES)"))
 (segment (start 167 136) (end 169.5 133.5) (width 0.2) (layer "F.Cu") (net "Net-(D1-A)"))
 (segment (start 170.455 133.5) (end 175.27 138.315) (width 0.2) (layer "F.Cu") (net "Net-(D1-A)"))
 (segment (start 169.5 133.5) (end 170.455 133.5) (width 0.2) (layer "F.Cu") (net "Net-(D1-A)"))
 (segment (start 173.872793 124.1) (end 150.399999 124.1) (width 0.2) (layer "F.Cu") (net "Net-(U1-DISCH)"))
 (segment (start 151.524448 131.5) (end 168.272793 131.5) (width 0.2) (layer "F.Cu") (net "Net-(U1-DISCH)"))
 (segment (start 137.595 132.414214) (end 137.595 131.585786) (width 0.2) (layer "F.Cu") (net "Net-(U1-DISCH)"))
 (segment (start 139.495 131) (end 140.495 132) (width 0.2) (layer "F.Cu") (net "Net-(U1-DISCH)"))
 (segment (start 138.185786 125.185786) (end 139 126) (width 0.2) (layer "F.Cu") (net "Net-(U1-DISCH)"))
 (segment (start 142.54 129.955) (end 142.54 125.585786) (width 0.2) (layer "F.Cu") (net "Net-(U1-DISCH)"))
 (segment (start 174.4 124.627207) (end 173.872793 124.1) (width 0.2) (layer "F.Cu") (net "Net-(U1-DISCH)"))
 (segment (start 150.95 134.96) (end 150.604448 134.96) (width 0.2) (layer "F.Cu") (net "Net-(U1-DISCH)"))
 (segment (start 174.4 125.372793) (end 174.4 124.627207) (width 0.2) (layer "F.Cu") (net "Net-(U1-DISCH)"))
 (segment (start 150.96 134.96) (end 151 135) (width 0.2) (layer "F.Cu") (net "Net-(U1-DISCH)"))
 (segment (start 150.604448 134.96) (end 149.675 134.030552) (width 0.2) (layer "F.Cu") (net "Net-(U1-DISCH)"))
 (segment (start 138.180786 131) (end 139.495 131) (width 0.2) (layer "F.Cu") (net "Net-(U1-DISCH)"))
 (segment (start 141.554214 124.6) (end 138.420101 124.6) (width 0.2) (layer "F.Cu") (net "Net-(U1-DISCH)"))
 (segment (start 149.675 133.349448) (end 151.524448 131.5) (width 0.2) (layer "F.Cu") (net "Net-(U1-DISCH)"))
 (segment (start 168.272793 131.5) (end 174.4 125.372793) (width 0.2) (layer "F.Cu") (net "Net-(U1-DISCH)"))
 (segment (start 149.675 134.030552) (end 149.675 133.349448) (width 0.2) (layer "F.Cu") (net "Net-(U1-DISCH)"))
 (segment (start 150.95 134.96) (end 150.96 134.96) (width 0.2) (layer "F.Cu") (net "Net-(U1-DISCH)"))
 (segment (start 142.54 125.585786) (end 141.554214 124.6) (width 0.2) (layer "F.Cu") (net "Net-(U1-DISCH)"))
 (segment (start 138.420101 124.6) (end 138.185786 124.834315) (width 0.2) (layer "F.Cu") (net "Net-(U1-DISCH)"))
 (segment (start 140.699997 133.8) (end 138.980786 133.8) (width 0.2) (layer "F.Cu") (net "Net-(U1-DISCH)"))
 (segment (start 150.399999 124.1) (end 140.699997 133.8) (width 0.2) (layer "F.Cu") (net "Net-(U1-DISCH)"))
 (segment (start 138.185786 124.834315) (end 138.185786 125.185786) (width 0.2) (layer "F.Cu") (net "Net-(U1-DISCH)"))
 (segment (start 137.595 131.585786) (end 138.180786 131) (width 0.2) (layer "F.Cu") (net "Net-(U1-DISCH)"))
 (segment (start 140.495 132) (end 142.54 129.955) (width 0.2) (layer "F.Cu") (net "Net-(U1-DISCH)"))
 (segment (start 138.980786 133.8) (end 137.595 132.414214) (width 0.2) (layer "F.Cu") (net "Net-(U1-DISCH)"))
 (segment (start 138.595 132) (end 139.995 133.4) (width 0.2) (layer "F.Cu") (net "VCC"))
 (segment (start 140.534311 133.4) (end 152.834314 121.1) (width 0.2) (layer "F.Cu") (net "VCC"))
 (segment (start 175.9 126.665686) (end 170.665685 131.9) (width 0.2) (layer "F.Cu") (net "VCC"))
 (segment (start 152.225 135.775) (end 152.167776 135.832224) (width 0.2) (layer "F.Cu") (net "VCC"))
 (segment (start 158.731238 131.9) (end 154.065619 136.565619) (width 0.2) (layer "F.Cu") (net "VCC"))
 (segment (start 139.995 133.4) (end 140.534311 133.4) (width 0.2) (layer "F.Cu") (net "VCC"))
 (segment (start 148.768762 137.5) (end 146 137.5) (width 0.2) (layer "F.Cu") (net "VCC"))
 (segment (start 173.165685 121.1) (end 175.9 123.834315) (width 0.2) (layer "F.Cu") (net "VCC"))
 (segment (start 170.665685 131.9) (end 158.731238 131.9) (width 0.2) (layer "F.Cu") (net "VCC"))
 (segment (start 175.9 123.834315) (end 175.9 126.665686) (width 0.2) (layer "F.Cu") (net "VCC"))
 (segment (start 149.768762 138.5) (end 148.768762 137.5) (width 0.2) (layer "F.Cu") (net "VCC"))
 (segment (start 152.131237 138.5) (end 149.768762 138.5) (width 0.2) (layer "F.Cu") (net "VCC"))
 (segment (start 152.225 134.619448) (end 152.225 135.775) (width 0.2) (layer "F.Cu") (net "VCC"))
 (segment (start 152.901171 136.565619) (end 154.065619 136.565619) (width 0.2) (layer "F.Cu") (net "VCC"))
 (segment (start 150.95 133.69) (end 151.295552 133.69) (width 0.2) (layer "F.Cu") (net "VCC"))
 (segment (start 151.295552 133.69) (end 152.225 134.619448) (width 0.2) (layer "F.Cu") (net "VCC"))
 (segment (start 152.834314 121.1) (end 173.165685 121.1) (width 0.2) (layer "F.Cu") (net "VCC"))
 (segment (start 152.167776 135.832224) (end 152.901171 136.565619) (width 0.2) (layer "F.Cu") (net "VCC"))
 (segment (start 154.065619 136.565619) (end 152.131237 138.5) (width 0.2) (layer "F.Cu") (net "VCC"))
 (segment (start 145.65162 136.23) (end 146 136.23) (width 0.2) (layer "F.Cu") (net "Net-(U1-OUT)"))
 (segment (start 144.984448 138.1) (end 144.725 137.840552) (width 0.2) (layer "F.Cu") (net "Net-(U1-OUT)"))
 (segment (start 159.020001 138.899999) (end 149.603076 138.9) (width 0.2) (layer "F.Cu") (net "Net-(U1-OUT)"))
 (segment (start 161.92 136) (end 159.020001 138.899999) (width 0.2) (layer "F.Cu") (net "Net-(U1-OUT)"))
 (segment (start 144.725 137.15662) (end 145.65162 136.23) (width 0.2) (layer "F.Cu") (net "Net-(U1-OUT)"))
 (segment (start 149.603076 138.9) (end 148.803077 138.1) (width 0.2) (layer "F.Cu") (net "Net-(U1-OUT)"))
 (segment (start 148.803077 138.1) (end 144.984448 138.1) (width 0.2) (layer "F.Cu") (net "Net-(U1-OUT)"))
 (segment (start 144.725 137.840552) (end 144.725 137.15662) (width 0.2) (layer "F.Cu") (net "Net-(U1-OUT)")))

